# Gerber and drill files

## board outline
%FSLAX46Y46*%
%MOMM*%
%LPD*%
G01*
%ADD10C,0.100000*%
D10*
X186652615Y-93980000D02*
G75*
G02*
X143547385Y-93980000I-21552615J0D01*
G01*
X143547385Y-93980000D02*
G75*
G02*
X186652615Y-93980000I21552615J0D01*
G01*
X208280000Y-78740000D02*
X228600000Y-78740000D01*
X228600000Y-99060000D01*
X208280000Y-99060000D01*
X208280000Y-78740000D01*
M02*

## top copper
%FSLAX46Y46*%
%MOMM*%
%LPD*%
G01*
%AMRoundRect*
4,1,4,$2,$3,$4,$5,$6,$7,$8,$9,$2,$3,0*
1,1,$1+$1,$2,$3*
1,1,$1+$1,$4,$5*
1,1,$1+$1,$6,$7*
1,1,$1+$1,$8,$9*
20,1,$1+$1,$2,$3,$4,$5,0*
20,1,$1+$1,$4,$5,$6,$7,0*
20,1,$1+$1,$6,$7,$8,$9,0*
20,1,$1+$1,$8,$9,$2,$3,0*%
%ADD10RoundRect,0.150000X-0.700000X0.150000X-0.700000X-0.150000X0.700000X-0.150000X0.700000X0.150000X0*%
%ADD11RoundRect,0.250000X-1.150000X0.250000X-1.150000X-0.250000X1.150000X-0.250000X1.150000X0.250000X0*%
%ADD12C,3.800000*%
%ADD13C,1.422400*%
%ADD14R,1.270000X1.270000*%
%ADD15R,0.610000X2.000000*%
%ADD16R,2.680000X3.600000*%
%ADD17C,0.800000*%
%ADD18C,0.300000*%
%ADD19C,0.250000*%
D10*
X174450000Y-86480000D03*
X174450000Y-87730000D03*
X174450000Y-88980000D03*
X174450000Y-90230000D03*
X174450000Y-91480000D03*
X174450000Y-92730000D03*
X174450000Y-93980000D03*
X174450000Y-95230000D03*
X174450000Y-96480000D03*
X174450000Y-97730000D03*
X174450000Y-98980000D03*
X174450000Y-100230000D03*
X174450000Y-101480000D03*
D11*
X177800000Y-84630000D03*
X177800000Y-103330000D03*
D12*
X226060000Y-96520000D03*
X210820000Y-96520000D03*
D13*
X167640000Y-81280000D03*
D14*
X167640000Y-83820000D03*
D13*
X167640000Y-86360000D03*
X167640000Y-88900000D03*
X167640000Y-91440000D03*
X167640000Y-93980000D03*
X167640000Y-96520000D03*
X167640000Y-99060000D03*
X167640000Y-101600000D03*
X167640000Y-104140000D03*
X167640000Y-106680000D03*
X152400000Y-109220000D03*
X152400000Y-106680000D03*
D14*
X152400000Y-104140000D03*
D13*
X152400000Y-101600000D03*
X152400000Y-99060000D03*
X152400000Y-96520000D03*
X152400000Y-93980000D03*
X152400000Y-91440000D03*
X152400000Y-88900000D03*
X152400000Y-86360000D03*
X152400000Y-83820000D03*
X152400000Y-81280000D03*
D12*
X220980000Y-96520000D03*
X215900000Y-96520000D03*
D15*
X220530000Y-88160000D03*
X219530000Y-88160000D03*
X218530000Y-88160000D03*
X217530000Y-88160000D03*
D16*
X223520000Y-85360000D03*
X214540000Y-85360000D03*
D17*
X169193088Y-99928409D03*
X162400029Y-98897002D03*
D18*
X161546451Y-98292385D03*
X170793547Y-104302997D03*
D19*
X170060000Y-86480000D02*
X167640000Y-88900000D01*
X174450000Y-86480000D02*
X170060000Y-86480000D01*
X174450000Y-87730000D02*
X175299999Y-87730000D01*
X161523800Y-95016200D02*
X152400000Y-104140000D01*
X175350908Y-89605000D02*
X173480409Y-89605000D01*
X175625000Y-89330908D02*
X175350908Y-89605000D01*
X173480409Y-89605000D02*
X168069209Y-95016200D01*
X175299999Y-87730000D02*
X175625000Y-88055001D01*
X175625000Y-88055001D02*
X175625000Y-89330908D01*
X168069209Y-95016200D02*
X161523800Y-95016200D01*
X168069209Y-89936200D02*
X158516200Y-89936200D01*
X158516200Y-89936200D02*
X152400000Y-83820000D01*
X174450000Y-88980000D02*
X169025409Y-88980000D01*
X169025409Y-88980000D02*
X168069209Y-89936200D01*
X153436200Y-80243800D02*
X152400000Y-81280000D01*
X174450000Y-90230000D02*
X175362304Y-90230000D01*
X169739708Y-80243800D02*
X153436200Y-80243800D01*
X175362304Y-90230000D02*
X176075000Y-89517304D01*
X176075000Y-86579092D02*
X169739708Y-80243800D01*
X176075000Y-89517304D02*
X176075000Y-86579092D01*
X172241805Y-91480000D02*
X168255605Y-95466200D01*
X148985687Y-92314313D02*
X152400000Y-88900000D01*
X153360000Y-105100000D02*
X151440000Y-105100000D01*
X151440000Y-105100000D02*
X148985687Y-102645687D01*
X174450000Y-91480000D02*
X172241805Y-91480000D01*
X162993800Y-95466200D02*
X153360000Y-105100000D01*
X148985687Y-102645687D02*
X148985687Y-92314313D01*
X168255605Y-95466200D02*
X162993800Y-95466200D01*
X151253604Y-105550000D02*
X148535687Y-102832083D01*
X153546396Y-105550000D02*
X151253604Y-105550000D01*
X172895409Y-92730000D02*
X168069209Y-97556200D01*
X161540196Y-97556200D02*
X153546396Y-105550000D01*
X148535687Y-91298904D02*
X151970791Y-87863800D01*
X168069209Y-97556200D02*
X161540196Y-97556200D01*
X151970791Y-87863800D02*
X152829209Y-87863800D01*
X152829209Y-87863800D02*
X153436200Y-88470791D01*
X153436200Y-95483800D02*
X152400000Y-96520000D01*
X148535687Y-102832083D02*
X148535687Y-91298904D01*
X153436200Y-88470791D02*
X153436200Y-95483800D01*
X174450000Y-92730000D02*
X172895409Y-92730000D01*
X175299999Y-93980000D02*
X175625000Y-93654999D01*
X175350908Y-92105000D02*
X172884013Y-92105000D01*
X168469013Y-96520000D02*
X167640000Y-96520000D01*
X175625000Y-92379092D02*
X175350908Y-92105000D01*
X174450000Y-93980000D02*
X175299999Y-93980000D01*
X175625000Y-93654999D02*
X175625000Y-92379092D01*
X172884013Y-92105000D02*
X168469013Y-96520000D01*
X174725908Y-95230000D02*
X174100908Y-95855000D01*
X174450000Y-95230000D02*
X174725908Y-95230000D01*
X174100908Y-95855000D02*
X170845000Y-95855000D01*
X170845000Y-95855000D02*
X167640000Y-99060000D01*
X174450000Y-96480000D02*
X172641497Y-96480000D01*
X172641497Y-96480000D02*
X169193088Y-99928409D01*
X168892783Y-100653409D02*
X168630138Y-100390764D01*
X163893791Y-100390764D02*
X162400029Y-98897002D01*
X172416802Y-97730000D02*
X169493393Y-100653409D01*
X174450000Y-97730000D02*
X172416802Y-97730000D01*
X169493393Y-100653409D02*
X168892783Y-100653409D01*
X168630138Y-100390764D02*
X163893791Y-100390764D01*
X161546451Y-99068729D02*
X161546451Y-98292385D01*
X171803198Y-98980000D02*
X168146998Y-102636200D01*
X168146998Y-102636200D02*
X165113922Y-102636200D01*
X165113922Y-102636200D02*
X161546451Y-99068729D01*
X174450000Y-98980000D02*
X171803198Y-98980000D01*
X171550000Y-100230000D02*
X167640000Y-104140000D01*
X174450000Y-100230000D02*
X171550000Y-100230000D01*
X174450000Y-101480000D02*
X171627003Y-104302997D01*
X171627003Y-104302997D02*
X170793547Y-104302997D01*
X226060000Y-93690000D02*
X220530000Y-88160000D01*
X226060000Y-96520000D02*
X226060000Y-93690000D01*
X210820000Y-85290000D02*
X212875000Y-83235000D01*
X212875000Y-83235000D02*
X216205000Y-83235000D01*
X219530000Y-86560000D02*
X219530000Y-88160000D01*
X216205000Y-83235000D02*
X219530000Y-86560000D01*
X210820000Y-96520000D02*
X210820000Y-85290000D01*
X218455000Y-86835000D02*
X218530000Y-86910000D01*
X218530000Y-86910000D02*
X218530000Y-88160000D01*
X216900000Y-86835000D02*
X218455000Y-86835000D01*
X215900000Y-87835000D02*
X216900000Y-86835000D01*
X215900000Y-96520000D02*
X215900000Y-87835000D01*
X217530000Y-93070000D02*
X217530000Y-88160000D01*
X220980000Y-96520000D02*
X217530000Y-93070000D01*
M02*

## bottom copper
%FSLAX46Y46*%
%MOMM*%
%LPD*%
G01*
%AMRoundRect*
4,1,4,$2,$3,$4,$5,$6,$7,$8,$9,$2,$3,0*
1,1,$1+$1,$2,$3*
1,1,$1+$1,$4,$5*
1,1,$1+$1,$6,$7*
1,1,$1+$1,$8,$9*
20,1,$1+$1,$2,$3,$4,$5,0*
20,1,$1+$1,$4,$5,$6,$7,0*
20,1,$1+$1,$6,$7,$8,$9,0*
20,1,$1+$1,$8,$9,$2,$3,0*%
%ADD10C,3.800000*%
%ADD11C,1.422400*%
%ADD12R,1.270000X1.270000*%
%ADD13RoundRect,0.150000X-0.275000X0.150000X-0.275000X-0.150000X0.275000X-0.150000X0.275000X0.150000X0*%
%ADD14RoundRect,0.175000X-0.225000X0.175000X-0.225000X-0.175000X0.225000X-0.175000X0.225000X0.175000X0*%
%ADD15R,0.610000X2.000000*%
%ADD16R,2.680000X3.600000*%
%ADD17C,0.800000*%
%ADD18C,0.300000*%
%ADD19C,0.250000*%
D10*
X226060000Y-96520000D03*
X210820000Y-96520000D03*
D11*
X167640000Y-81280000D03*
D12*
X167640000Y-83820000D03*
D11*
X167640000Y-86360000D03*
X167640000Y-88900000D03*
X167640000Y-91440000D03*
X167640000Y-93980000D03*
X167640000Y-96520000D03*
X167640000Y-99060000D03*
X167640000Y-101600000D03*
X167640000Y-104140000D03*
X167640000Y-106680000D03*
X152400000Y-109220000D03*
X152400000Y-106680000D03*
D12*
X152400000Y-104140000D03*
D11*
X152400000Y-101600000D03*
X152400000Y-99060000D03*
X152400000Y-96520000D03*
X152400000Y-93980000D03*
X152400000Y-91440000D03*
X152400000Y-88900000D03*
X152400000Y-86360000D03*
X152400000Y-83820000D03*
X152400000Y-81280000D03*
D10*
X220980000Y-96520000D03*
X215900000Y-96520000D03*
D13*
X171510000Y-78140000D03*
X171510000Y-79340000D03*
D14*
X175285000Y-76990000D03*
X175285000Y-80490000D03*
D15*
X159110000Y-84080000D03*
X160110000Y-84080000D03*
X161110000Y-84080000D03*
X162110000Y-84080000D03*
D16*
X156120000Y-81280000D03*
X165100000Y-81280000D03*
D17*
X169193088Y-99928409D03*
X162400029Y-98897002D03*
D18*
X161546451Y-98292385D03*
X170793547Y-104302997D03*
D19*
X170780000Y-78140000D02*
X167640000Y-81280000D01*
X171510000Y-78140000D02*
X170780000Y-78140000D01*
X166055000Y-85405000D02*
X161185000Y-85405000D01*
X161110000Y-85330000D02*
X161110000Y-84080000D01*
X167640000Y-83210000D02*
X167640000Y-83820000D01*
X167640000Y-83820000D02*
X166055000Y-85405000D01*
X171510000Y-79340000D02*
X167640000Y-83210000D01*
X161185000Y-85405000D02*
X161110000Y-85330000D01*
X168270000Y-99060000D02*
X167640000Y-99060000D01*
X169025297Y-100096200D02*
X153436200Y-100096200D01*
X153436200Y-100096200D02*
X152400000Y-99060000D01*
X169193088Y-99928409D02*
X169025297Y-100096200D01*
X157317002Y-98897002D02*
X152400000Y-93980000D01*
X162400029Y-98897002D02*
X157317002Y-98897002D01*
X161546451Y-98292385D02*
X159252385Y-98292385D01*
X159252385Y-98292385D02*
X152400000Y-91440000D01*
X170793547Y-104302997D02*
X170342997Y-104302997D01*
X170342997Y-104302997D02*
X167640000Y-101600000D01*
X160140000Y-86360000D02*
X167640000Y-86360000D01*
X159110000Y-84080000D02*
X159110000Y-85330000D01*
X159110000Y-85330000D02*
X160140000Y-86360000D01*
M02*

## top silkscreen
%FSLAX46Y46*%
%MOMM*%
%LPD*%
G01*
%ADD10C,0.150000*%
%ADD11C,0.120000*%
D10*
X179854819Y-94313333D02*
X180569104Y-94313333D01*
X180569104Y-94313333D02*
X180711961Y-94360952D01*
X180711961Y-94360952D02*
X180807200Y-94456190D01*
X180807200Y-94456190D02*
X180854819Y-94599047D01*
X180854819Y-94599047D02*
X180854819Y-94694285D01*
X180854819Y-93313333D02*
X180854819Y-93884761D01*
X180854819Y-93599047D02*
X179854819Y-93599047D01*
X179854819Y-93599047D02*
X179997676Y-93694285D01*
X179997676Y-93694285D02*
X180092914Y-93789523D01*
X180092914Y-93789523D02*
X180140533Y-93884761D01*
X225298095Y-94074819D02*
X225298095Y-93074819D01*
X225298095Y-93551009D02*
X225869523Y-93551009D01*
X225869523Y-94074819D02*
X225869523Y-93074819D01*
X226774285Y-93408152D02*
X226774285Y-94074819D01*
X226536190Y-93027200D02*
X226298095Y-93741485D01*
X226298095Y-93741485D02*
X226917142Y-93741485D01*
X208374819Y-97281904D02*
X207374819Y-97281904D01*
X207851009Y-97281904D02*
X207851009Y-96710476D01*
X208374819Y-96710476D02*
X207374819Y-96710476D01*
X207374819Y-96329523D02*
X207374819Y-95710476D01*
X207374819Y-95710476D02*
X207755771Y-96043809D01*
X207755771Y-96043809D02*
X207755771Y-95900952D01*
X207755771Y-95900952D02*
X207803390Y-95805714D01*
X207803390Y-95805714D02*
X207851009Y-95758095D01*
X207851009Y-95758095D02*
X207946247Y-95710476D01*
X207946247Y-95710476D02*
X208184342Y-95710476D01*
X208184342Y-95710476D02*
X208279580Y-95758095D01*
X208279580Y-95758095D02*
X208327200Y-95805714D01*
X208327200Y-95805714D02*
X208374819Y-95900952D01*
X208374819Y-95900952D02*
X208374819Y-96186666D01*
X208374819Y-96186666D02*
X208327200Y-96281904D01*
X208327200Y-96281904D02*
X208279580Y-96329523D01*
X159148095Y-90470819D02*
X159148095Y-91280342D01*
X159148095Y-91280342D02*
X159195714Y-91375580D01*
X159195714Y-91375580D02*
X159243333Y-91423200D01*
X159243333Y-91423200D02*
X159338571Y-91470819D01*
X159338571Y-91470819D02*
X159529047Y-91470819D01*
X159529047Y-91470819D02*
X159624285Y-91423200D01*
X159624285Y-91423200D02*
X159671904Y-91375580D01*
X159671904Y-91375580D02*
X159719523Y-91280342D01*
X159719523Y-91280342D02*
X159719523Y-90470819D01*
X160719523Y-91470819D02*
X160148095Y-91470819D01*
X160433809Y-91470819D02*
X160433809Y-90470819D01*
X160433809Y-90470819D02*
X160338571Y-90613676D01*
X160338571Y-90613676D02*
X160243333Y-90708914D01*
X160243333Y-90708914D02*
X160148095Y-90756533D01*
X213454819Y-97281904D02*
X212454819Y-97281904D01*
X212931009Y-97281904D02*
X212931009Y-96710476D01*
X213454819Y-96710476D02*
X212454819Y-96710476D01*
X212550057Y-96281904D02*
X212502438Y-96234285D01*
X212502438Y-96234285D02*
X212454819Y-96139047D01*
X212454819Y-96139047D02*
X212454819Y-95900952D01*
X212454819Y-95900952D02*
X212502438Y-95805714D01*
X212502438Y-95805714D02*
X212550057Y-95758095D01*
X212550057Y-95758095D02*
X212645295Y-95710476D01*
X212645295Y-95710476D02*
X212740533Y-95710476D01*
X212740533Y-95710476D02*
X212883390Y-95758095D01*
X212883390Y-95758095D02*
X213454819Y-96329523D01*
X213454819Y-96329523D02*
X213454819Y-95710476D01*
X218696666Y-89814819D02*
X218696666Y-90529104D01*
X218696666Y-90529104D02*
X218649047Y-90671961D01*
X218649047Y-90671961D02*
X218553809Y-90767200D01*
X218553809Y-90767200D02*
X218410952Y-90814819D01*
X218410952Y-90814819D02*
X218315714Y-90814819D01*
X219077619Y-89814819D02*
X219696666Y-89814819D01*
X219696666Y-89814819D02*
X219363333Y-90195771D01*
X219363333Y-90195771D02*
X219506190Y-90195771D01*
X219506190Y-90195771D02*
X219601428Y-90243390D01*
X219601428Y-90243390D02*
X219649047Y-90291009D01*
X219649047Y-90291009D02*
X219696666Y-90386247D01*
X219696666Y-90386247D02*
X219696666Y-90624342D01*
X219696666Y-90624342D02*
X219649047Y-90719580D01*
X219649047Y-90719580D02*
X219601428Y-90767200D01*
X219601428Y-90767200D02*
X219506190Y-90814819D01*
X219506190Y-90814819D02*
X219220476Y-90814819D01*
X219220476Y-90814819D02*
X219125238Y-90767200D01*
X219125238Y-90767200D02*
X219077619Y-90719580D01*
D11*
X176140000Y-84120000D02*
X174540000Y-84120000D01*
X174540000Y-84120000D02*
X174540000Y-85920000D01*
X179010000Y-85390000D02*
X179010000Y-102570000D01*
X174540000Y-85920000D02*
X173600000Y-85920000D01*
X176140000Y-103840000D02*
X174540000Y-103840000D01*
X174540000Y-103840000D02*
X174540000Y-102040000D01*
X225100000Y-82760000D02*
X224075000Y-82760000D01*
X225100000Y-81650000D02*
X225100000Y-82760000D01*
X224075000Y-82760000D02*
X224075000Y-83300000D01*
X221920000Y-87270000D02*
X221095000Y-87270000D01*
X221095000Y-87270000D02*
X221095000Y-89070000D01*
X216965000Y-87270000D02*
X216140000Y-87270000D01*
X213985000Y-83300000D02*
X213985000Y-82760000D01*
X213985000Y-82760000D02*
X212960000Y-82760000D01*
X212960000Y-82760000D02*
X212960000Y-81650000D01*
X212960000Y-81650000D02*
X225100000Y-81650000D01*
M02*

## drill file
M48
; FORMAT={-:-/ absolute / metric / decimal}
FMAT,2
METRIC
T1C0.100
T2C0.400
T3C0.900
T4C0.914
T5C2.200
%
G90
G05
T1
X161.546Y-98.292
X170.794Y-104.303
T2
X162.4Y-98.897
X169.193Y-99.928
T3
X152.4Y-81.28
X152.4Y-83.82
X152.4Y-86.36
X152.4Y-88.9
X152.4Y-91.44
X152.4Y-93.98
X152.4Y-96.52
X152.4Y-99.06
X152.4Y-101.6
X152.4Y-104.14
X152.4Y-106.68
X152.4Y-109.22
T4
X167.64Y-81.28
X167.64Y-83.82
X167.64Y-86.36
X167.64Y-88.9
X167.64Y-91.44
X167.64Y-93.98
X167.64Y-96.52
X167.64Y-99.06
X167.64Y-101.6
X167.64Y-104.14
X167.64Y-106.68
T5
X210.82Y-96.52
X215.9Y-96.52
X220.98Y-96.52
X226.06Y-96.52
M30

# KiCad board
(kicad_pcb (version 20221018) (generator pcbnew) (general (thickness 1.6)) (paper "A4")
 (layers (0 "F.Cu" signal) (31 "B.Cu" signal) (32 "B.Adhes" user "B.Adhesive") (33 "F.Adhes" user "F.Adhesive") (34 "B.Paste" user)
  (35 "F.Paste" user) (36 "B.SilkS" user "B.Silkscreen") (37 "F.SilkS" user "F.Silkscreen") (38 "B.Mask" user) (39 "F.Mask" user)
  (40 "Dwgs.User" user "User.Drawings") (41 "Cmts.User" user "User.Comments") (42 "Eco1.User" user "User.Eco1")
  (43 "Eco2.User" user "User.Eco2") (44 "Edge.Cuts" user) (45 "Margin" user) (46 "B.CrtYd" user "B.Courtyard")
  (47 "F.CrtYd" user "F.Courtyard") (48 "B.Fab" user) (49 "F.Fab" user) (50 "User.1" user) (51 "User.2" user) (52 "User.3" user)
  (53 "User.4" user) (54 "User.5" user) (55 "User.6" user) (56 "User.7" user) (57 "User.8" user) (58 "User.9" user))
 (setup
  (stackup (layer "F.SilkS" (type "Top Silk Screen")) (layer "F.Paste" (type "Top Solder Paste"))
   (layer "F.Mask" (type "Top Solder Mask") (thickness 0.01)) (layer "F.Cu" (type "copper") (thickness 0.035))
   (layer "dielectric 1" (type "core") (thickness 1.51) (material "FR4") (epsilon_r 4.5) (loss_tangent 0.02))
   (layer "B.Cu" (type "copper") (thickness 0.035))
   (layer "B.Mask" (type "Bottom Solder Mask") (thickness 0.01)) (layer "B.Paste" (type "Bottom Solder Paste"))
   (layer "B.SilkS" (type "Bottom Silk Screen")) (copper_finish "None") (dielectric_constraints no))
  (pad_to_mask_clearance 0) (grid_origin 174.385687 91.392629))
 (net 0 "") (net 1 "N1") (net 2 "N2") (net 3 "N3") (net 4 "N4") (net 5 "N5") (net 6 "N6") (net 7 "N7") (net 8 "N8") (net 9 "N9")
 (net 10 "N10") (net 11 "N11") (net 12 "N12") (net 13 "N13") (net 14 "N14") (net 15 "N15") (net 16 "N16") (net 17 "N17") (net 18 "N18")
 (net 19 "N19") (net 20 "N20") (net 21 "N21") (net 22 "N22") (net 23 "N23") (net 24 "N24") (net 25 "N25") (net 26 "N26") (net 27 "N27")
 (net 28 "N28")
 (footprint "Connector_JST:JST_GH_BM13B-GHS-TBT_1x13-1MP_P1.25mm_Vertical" (layer "F.Cu") (at 176.4 93.98 -90)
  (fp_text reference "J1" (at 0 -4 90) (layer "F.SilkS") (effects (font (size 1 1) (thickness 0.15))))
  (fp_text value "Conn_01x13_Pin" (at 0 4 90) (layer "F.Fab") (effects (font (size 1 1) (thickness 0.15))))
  (fp_line (start -9.86 0.26) (end -9.86 1.86) (stroke (width 0.12) (type solid)) (layer "F.SilkS"))
  (fp_line (start -9.86 1.86) (end -8.06 1.86) (stroke (width 0.12) (type solid)) (layer "F.SilkS"))
  (fp_line (start -8.59 -2.61) (end 8.59 -2.61) (stroke (width 0.12) (type solid)) (layer "F.SilkS"))
  (fp_line (start -8.06 1.86) (end -8.06 2.8) (stroke (width 0.12) (type solid)) (layer "F.SilkS"))
  (fp_line (start 9.86 0.26) (end 9.86 1.86) (stroke (width 0.12) (type solid)) (layer "F.SilkS"))
  (fp_line (start 9.86 1.86) (end 8.06 1.86) (stroke (width 0.12) (type solid)) (layer "F.SilkS"))
  (pad "1" smd roundrect (at -7.5 1.95 270) (size 0.6 1.7) (layers "F.Cu" "F.Paste" "F.Mask") (roundrect_rratio 0.25) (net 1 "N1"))
  (pad "2" smd roundrect (at -6.25 1.95 270) (size 0.6 1.7) (layers "F.Cu" "F.Paste" "F.Mask") (roundrect_rratio 0.25) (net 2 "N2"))
  (pad "3" smd roundrect (at -5 1.95 270) (size 0.6 1.7) (layers "F.Cu" "F.Paste" "F.Mask") (roundrect_rratio 0.25) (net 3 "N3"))
  (pad "4" smd roundrect (at -3.75 1.95 270) (size 0.6 1.7) (layers "F.Cu" "F.Paste" "F.Mask") (roundrect_rratio 0.25) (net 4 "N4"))
  (pad "5" smd roundrect (at -2.5 1.95 270) (size 0.6 1.7) (layers "F.Cu" "F.Paste" "F.Mask") (roundrect_rratio 0.25) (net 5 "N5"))
  (pad "6" smd roundrect (at -1.25 1.95 270) (size 0.6 1.7) (layers "F.Cu" "F.Paste" "F.Mask") (roundrect_rratio 0.25) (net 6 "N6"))
  (pad "7" smd roundrect (at 0 1.95 270) (size 0.6 1.7) (layers "F.Cu" "F.Paste" "F.Mask") (roundrect_rratio 0.25) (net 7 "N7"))
  (pad "8" smd roundrect (at 1.25 1.95 270) (size 0.6 1.7) (layers "F.Cu" "F.Paste" "F.Mask") (roundrect_rratio 0.25) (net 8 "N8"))
  (pad "9" smd roundrect (at 2.5 1.95 270) (size 0.6 1.7) (layers "F.Cu" "F.Paste" "F.Mask") (roundrect_rratio 0.25) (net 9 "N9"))
  (pad "10" smd roundrect (at 3.75 1.95 270) (size 0.6 1.7) (layers "F.Cu" "F.Paste" "F.Mask") (roundrect_rratio 0.25) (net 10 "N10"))
  (pad "11" smd roundrect (at 5 1.95 270) (size 0.6 1.7) (layers "F.Cu" "F.Paste" "F.Mask") (roundrect_rratio 0.25) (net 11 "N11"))
  (pad "12" smd roundrect (at 6.25 1.95 270) (size 0.6 1.7) (layers "F.Cu" "F.Paste" "F.Mask") (roundrect_rratio 0.25) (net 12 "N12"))
  (pad "13" smd roundrect (at 7.5 1.95 270) (size 0.6 1.7) (layers "F.Cu" "F.Paste" "F.Mask") (roundrect_rratio 0.25) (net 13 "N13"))
  (pad "MP" smd roundrect (at -9.35 -1.4 270) (size 1 2.8) (layers "F.Cu" "F.Paste" "F.Mask") (roundrect_rratio 0.25))
  (pad "MP" smd roundrect (at 9.35 -1.4 270) (size 1 2.8) (layers "F.Cu" "F.Paste" "F.Mask") (roundrect_rratio 0.25)))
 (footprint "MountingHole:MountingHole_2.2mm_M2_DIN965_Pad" (layer "F.Cu") (at 226.06 96.52)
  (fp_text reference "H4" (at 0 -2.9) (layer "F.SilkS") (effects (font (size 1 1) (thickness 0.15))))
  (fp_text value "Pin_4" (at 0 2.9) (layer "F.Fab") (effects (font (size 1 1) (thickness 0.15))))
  (pad "1" thru_hole circle (at 0 0) (size 3.8 3.8) (drill 2.2) (layers "*.Cu" "*.Mask") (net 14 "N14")))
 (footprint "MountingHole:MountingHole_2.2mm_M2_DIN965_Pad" (layer "F.Cu") (at 210.82 96.52 90)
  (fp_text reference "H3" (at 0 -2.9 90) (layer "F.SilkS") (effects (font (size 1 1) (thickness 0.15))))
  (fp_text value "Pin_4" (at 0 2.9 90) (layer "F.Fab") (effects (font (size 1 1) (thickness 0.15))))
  (pad "1" thru_hole circle (at 0 0 90) (size 3.8 3.8) (drill 2.2) (layers "*.Cu" "*.Mask") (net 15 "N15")))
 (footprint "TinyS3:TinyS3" (layer "F.Cu") (at 159.91 95.216)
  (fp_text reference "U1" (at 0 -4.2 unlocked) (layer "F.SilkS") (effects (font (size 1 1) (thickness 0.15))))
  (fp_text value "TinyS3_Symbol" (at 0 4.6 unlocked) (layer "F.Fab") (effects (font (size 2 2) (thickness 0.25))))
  (pad "1" thru_hole circle (at 7.73 -13.936) (size 1.4224 1.4224) (drill 0.9144) (layers "*.Cu" "*.Mask") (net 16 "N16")
   (solder_mask_margin 0.0254))
  (pad "2" thru_hole rect (at 7.73 -11.396) (size 1.27 1.27) (drill 0.9144) (layers "*.Cu" "*.Mask") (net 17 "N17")
   (solder_mask_margin 0.0254))
  (pad "3" thru_hole circle (at 7.73 -8.856) (size 1.4224 1.4224) (drill 0.9144) (layers "*.Cu" "*.Mask") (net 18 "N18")
   (solder_mask_margin 0.0254))
  (pad "4" thru_hole circle (at 7.73 -6.316) (size 1.4224 1.4224) (drill 0.9144) (layers "*.Cu" "*.Mask") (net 1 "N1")
   (solder_mask_margin 0.0254))
  (pad "5" thru_hole circle (at 7.73 -3.776) (size 1.4224 1.4224) (drill 0.9144) (layers "*.Cu" "*.Mask") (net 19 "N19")
   (solder_mask_margin 0.0254))
  (pad "6" thru_hole circle (at 7.73 -1.236) (size 1.4224 1.4224) (drill 0.9144) (layers "*.Cu" "*.Mask") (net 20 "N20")
   (solder_mask_margin 0.0254))
  (pad "7" thru_hole circle (at 7.73 1.304) (size 1.4224 1.4224) (drill 0.9144) (layers "*.Cu" "*.Mask") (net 7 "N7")
   (solder_mask_margin 0.0254))
  (pad "8" thru_hole circle (at 7.73 3.844) (size 1.4224 1.4224) (drill 0.9144) (layers "*.Cu" "*.Mask") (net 8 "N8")
   (solder_mask_margin 0.0254))
  (pad "9" thru_hole circle (at 7.73 6.384) (size 1.4224 1.4224) (drill 0.9144) (layers "*.Cu" "*.Mask") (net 13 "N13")
   (solder_mask_margin 0.0254))
  (pad "10" thru_hole circle (at 7.73 8.924) (size 1.4224 1.4224) (drill 0.9144) (layers "*.Cu" "*.Mask") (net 12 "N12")
   (solder_mask_margin 0.0254))
  (pad "11" thru_hole circle (at 7.73 11.464) (size 1.4224 1.4224) (drill 0.9144) (layers "*.Cu" "*.Mask") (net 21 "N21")
   (solder_mask_margin 0.0254))
  (pad "12" thru_hole circle (at -7.51 14.004) (size 1.4224 1.4224) (drill 0.9) (layers "*.Cu" "*.Mask") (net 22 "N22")
   (solder_mask_margin 0.0254))
  (pad "13" thru_hole circle (at -7.51 11.464) (size 1.4224 1.4224) (drill 0.9) (layers "*.Cu" "*.Mask") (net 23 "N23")
   (solder_mask_margin 0.0254))
  (pad "14" thru_hole rect (at -7.51 8.924) (size 1.27 1.27) (drill 0.9) (layers "*.Cu" "*.Mask") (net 2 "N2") (solder_mask_margin 0.0254))
  (pad "15" thru_hole circle (at -7.51 6.384) (size 1.4224 1.4224) (drill 0.9) (layers "*.Cu" "*.Mask") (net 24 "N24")
   (solder_mask_margin 0.0254))
  (pad "16" thru_hole circle (at -7.51 3.844) (size 1.4224 1.4224) (drill 0.9) (layers "*.Cu" "*.Mask") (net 9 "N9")
   (solder_mask_margin 0.0254))
  (pad "17" thru_hole circle (at -7.51 1.304) (size 1.4224 1.4224) (drill 0.9) (layers "*.Cu" "*.Mask") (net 6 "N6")
   (solder_mask_margin 0.0254))
  (pad "18" thru_hole circle (at -7.51 -1.236) (size 1.4224 1.4224) (drill 0.9) (layers "*.Cu" "*.Mask") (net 10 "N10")
   (solder_mask_margin 0.0254))
  (pad "19" thru_hole circle (at -7.51 -3.776) (size 1.4224 1.4224) (drill 0.9) (layers "*.Cu" "*.Mask") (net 11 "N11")
   (solder_mask_margin 0.0254))
  (pad "20" thru_hole circle (at -7.51 -6.316) (size 1.4224 1.4224) (drill 0.9) (layers "*.Cu" "*.Mask") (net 5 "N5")
   (solder_mask_margin 0.0254))
  (pad "21" thru_hole circle (at -7.51 -8.856) (size 1.4224 1.4224) (drill 0.9) (layers "*.Cu" "*.Mask") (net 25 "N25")
   (solder_mask_margin 0.0254))
  (pad "22" thru_hole circle (at -7.51 -11.396) (size 1.4224 1.4224) (drill 0.9) (layers "*.Cu" "*.Mask") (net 3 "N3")
   (solder_mask_margin 0.0254))
  (pad "23" thru_hole circle (at -7.51 -13.936) (size 1.4224 1.4224) (drill 0.9) (layers "*.Cu" "*.Mask") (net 4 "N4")
   (solder_mask_margin 0.0254)))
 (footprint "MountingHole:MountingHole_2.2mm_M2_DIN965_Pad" (layer "F.Cu") (at 220.98 96.52 90)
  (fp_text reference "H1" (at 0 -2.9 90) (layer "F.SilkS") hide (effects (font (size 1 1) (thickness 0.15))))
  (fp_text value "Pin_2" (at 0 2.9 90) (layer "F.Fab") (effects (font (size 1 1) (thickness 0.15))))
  (pad "1" thru_hole circle (at 0 0 90) (size 3.8 3.8) (drill 2.2) (layers "*.Cu" "*.Mask") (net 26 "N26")))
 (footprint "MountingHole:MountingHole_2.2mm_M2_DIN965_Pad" (layer "F.Cu") (at 215.9 96.52 90)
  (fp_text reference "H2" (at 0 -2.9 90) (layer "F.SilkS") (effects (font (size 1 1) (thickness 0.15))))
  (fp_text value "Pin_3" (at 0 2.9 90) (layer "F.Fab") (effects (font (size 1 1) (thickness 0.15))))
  (pad "1" thru_hole circle (at 0 0 90) (size 3.8 3.8) (drill 2.2) (layers "*.Cu" "*.Mask") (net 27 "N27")))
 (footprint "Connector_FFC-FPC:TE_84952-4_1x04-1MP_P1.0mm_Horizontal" (layer "F.Cu") (at 219.03 86.36 180)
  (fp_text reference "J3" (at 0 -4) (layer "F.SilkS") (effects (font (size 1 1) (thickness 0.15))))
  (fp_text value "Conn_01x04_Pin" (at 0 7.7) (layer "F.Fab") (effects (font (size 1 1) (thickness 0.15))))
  (fp_line (start -6.07 3.6) (end -5.045 3.6) (stroke (width 0.12) (type solid)) (layer "F.SilkS"))
  (fp_line (start -6.07 4.71) (end -6.07 3.6) (stroke (width 0.12) (type solid)) (layer "F.SilkS"))
  (fp_line (start -5.045 3.6) (end -5.045 3.06) (stroke (width 0.12) (type solid)) (layer "F.SilkS"))
  (fp_line (start -2.89 -0.91) (end -2.065 -0.91) (stroke (width 0.12) (type solid)) (layer "F.SilkS"))
  (fp_line (start -2.065 -0.91) (end -2.065 -2.71) (stroke (width 0.12) (type solid)) (layer "F.SilkS"))
  (fp_line (start 2.065 -0.91) (end 2.89 -0.91) (stroke (width 0.12) (type solid)) (layer "F.SilkS"))
  (fp_line (start 5.045 3.06) (end 5.045 3.6) (stroke (width 0.12) (type solid)) (layer "F.SilkS"))
  (fp_line (start 5.045 3.6) (end 6.07 3.6) (stroke (width 0.12) (type solid)) (layer "F.SilkS"))
  (fp_line (start 6.07 3.6) (end 6.07 4.71) (stroke (width 0.12) (type solid)) (layer "F.SilkS"))
  (fp_line (start 6.07 4.71) (end -6.07 4.71) (stroke (width 0.12) (type solid)) (layer "F.SilkS"))
  (pad "1" smd rect (at -1.5 -1.8 180) (size 0.61 2) (layers "F.Cu" "F.Paste" "F.Mask") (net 14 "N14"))
  (pad "2" smd rect (at -0.5 -1.8 180) (size 0.61 2) (layers "F.Cu" "F.Paste" "F.Mask") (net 15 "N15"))
  (pad "3" smd rect (at 0.5 -1.8 180) (size 0.61 2) (layers "F.Cu" "F.Paste" "F.Mask") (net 27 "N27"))
  (pad "4" smd rect (at 1.5 -1.8 180) (size 0.61 2) (layers "F.Cu" "F.Paste" "F.Mask") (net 26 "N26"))
  (pad "MP" smd rect (at -4.49 1 180) (size 2.68 3.6) (layers "F.Cu" "F.Paste" "F.Mask"))
  (pad "MP" smd rect (at 4.49 1 180) (size 2.68 3.6) (layers "F.Cu" "F.Paste" "F.Mask")))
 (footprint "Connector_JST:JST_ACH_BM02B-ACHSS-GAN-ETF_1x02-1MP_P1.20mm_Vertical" (layer "B.Cu") (at 173.385 78.74 -90)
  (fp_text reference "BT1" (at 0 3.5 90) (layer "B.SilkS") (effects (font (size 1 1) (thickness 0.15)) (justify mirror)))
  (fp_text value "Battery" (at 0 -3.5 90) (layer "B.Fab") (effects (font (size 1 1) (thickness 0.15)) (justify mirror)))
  (pad "1" smd roundrect (at -0.6 1.875 270) (size 0.6 0.85) (layers "B.Cu" "B.Paste" "B.Mask") (roundrect_rratio 0.25) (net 16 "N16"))
  (pad "2" smd roundrect (at 0.6 1.875 270) (size 0.6 0.85) (layers "B.Cu" "B.Paste" "B.Mask") (roundrect_rratio 0.25) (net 17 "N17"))
  (pad "MP" smd roundrect (at -1.75 -1.9 270) (size 0.7 0.8) (layers "B.Cu" "B.Paste" "B.Mask") (roundrect_rratio 0.25))
  (pad "MP" smd roundrect (at 1.75 -1.9 270) (size 0.7 0.8) (layers "B.Cu" "B.Paste" "B.Mask") (roundrect_rratio 0.25)))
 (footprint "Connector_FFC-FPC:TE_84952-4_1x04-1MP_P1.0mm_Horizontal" (layer "B.Cu") (at 160.61 82.28)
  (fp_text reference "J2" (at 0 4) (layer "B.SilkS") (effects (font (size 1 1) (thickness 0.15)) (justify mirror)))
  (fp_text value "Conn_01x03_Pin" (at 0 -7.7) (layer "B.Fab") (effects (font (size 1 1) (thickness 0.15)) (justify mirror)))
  (pad "1" smd rect (at -1.5 1.8) (size 0.61 2) (layers "B.Cu" "B.Paste" "B.Mask") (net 18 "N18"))
  (pad "2" smd rect (at -0.5 1.8) (size 0.61 2) (layers "B.Cu" "B.Paste" "B.Mask") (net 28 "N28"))
  (pad "3" smd rect (at 0.5 1.8) (size 0.61 2) (layers "B.Cu" "B.Paste" "B.Mask") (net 17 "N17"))
  (pad "4" smd rect (at 1.5 1.8) (size 0.61 2) (layers "B.Cu" "B.Paste" "B.Mask"))
  (pad "MP" smd rect (at -4.49 -1) (size 2.68 3.6) (layers "B.Cu" "B.Paste" "B.Mask"))
  (pad "MP" smd rect (at 4.49 -1) (size 2.68 3.6) (layers "B.Cu" "B.Paste" "B.Mask")))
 (gr_circle (center 165.1 93.98) (end 180.34 78.74) (stroke (width 0.1) (type default)) (fill none) (layer "Edge.Cuts"))
 (gr_rect (start 208.28 78.74) (end 228.6 99.06) (stroke (width 0.1) (type default)) (fill none) (layer "Edge.Cuts"))
 (segment (start 170.78 78.14) (end 167.64 81.28) (width 0.25) (layer "B.Cu") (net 16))
 (segment (start 171.51 78.14) (end 170.78 78.14) (width 0.25) (layer "B.Cu") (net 16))
 (segment (start 166.055 85.405) (end 161.185 85.405) (width 0.25) (layer "B.Cu") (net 17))
 (segment (start 161.11 85.33) (end 161.11 84.08) (width 0.25) (layer "B.Cu") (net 17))
 (segment (start 167.64 83.21) (end 167.64 83.82) (width 0.25) (layer "B.Cu") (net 17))
 (segment (start 167.64 83.82) (end 166.055 85.405) (width 0.25) (layer "B.Cu") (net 17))
 (segment (start 171.51 79.34) (end 167.64 83.21) (width 0.25) (layer "B.Cu") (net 17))
 (segment (start 161.185 85.405) (end 161.11 85.33) (width 0.25) (layer "B.Cu") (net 17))
 (segment (start 170.06 86.48) (end 167.64 88.9) (width 0.25) (layer "F.Cu") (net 1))
 (segment (start 174.45 86.48) (end 170.06 86.48) (width 0.25) (layer "F.Cu") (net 1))
 (segment (start 174.45 87.73) (end 175.299999 87.73) (width 0.25) (layer "F.Cu") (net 2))
 (segment (start 161.5238 95.0162) (end 152.4 104.14) (width 0.25) (layer "F.Cu") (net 2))
 (segment (start 175.350908 89.605) (end 173.480409 89.605) (width 0.25) (layer "F.Cu") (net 2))
 (segment (start 175.625 89.330908) (end 175.350908 89.605) (width 0.25) (layer "F.Cu") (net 2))
 (segment (start 173.480409 89.605) (end 168.069209 95.0162) (width 0.25) (layer "F.Cu") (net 2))
 (segment (start 175.299999 87.73) (end 175.625 88.055001) (width 0.25) (layer "F.Cu") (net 2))
 (segment (start 175.625 88.055001) (end 175.625 89.330908) (width 0.25) (layer "F.Cu") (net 2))
 (segment (start 168.069209 95.0162) (end 161.5238 95.0162) (width 0.25) (layer "F.Cu") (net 2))
 (segment (start 168.069209 89.9362) (end 158.5162 89.9362) (width 0.25) (layer "F.Cu") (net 3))
 (segment (start 158.5162 89.9362) (end 152.4 83.82) (width 0.25) (layer "F.Cu") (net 3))
 (segment (start 174.45 88.98) (end 169.025409 88.98) (width 0.25) (layer "F.Cu") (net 3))
 (segment (start 169.025409 88.98) (end 168.069209 89.9362) (width 0.25) (layer "F.Cu") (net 3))
 (segment (start 153.4362 80.2438) (end 152.4 81.28) (width 0.25) (layer "F.Cu") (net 4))
 (segment (start 174.45 90.23) (end 175.362304 90.23) (width 0.25) (layer "F.Cu") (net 4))
 (segment (start 169.739708 80.2438) (end 153.4362 80.2438) (width 0.25) (layer "F.Cu") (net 4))
 (segment (start 175.362304 90.23) (end 176.075 89.517304) (width 0.25) (layer "F.Cu") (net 4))
 (segment (start 176.075 86.579092) (end 169.739708 80.2438) (width 0.25) (layer "F.Cu") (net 4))
 (segment (start 176.075 89.517304) (end 176.075 86.579092) (width 0.25) (layer "F.Cu") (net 4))
 (segment (start 172.241805 91.48) (end 168.255605 95.4662) (width 0.25) (layer "F.Cu") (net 5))
 (segment (start 148.985687 92.314313) (end 152.4 88.9) (width 0.25) (layer "F.Cu") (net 5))
 (segment (start 153.36 105.1) (end 151.44 105.1) (width 0.25) (layer "F.Cu") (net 5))
 (segment (start 151.44 105.1) (end 148.985687 102.645687) (width 0.25) (layer "F.Cu") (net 5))
 (segment (start 174.45 91.48) (end 172.241805 91.48) (width 0.25) (layer "F.Cu") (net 5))
 (segment (start 162.9938 95.4662) (end 153.36 105.1) (width 0.25) (layer "F.Cu") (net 5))
 (segment (start 148.985687 102.645687) (end 148.985687 92.314313) (width 0.25) (layer "F.Cu") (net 5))
 (segment (start 168.255605 95.4662) (end 162.9938 95.4662) (width 0.25) (layer "F.Cu") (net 5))
 (segment (start 151.253604 105.55) (end 148.535687 102.832083) (width 0.25) (layer "F.Cu") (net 6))
 (segment (start 153.546396 105.55) (end 151.253604 105.55) (width 0.25) (layer "F.Cu") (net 6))
 (segment (start 172.895409 92.73) (end 168.069209 97.5562) (width 0.25) (layer "F.Cu") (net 6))
 (segment (start 161.540196 97.5562) (end 153.546396 105.55) (width 0.25) (layer "F.Cu") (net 6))
 (segment (start 148.535687 91.298904) (end 151.970791 87.8638) (width 0.25) (layer "F.Cu") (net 6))
 (segment (start 168.069209 97.5562) (end 161.540196 97.5562) (width 0.25) (layer "F.Cu") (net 6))
 (segment (start 151.970791 87.8638) (end 152.829209 87.8638) (width 0.25) (layer "F.Cu") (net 6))
 (segment (start 152.829209 87.8638) (end 153.4362 88.470791) (width 0.25) (layer "F.Cu") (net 6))
 (segment (start 153.4362 95.4838) (end 152.4 96.52) (width 0.25) (layer "F.Cu") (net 6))
 (segment (start 148.535687 102.832083) (end 148.535687 91.298904) (width 0.25) (layer "F.Cu") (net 6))
 (segment (start 153.4362 88.470791) (end 153.4362 95.4838) (width 0.25) (layer "F.Cu") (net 6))
 (segment (start 174.45 92.73) (end 172.895409 92.73) (width 0.25) (layer "F.Cu") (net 6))
 (segment (start 175.299999 93.98) (end 175.625 93.654999) (width 0.25) (layer "F.Cu") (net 7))
 (segment (start 175.350908 92.105) (end 172.884013 92.105) (width 0.25) (layer "F.Cu") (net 7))
 (segment (start 168.469013 96.52) (end 167.64 96.52) (width 0.25) (layer "F.Cu") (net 7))
 (segment (start 175.625 92.379092) (end 175.350908 92.105) (width 0.25) (layer "F.Cu") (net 7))
 (segment (start 174.45 93.98) (end 175.299999 93.98) (width 0.25) (layer "F.Cu") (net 7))
 (segment (start 175.625 93.654999) (end 175.625 92.379092) (width 0.25) (layer "F.Cu") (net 7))
 (segment (start 172.884013 92.105) (end 168.469013 96.52) (width 0.25) (layer "F.Cu") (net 7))
 (segment (start 174.725908 95.23) (end 174.100908 95.855) (width 0.25) (layer "F.Cu") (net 8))
 (segment (start 174.45 95.23) (end 174.725908 95.23) (width 0.25) (layer "F.Cu") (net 8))
 (segment (start 174.100908 95.855) (end 170.845 95.855) (width 0.25) (layer "F.Cu") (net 8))
 (segment (start 170.845 95.855) (end 167.64 99.06) (width 0.25) (layer "F.Cu") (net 8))
 (segment (start 168.27 99.06) (end 167.64 99.06) (width 0.25) (layer "B.Cu") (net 8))
 (segment (start 174.45 96.48) (end 172.641497 96.48) (width 0.25) (layer "F.Cu") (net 9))
 (segment (start 172.641497 96.48) (end 169.193088 99.928409) (width 0.25) (layer "F.Cu") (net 9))
 (via (at 169.193088 99.928409) (size 0.8) (drill 0.4) (layers "F.Cu" "B.Cu") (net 9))
 (segment (start 169.025297 100.0962) (end 153.4362 100.0962) (width 0.25) (layer "B.Cu") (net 9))
 (segment (start 153.4362 100.0962) (end 152.4 99.06) (width 0.25) (layer "B.Cu") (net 9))
 (segment (start 169.193088 99.928409) (end 169.025297 100.0962) (width 0.25) (layer "B.Cu") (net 9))
 (segment (start 168.892783 100.653409) (end 168.630138 100.390764) (width 0.25) (layer "F.Cu") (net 10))
 (segment (start 163.893791 100.390764) (end 162.400029 98.897002) (width 0.25) (layer "F.Cu") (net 10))
 (segment (start 172.416802 97.73) (end 169.493393 100.653409) (width 0.25) (layer "F.Cu") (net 10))
 (segment (start 174.45 97.73) (end 172.416802 97.73) (width 0.25) (layer "F.Cu") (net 10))
 (segment (start 169.493393 100.653409) (end 168.892783 100.653409) (width 0.25) (layer "F.Cu") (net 10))
 (segment (start 168.630138 100.390764) (end 163.893791 100.390764) (width 0.25) (layer "F.Cu") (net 10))
 (via (at 162.400029 98.897002) (size 0.8) (drill 0.4) (layers "F.Cu" "B.Cu") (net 10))
 (segment (start 157.317002 98.897002) (end 152.4 93.98) (width 0.25) (layer "B.Cu") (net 10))
 (segment (start 162.400029 98.897002) (end 157.317002 98.897002) (width 0.25) (layer "B.Cu") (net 10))
 (segment (start 161.546451 99.068729) (end 161.546451 98.292385) (width 0.25) (layer "F.Cu") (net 11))
 (segment (start 171.803198 98.98) (end 168.146998 102.6362) (width 0.25) (layer "F.Cu") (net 11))
 (segment (start 168.146998 102.6362) (end 165.113922 102.6362) (width 0.25) (layer "F.Cu") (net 11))
 (segment (start 165.113922 102.6362) (end 161.546451 99.068729) (width 0.25) (layer "F.Cu") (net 11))
 (segment (start 174.45 98.98) (end 171.803198 98.98) (width 0.25) (layer "F.Cu") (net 11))
 (via micro (at 161.546451 98.292385) (size 0.3) (drill 0.1) (layers "F.Cu" "B.Cu") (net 11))
 (segment (start 161.546451 98.292385) (end 159.252385 98.292385) (width 0.25) (layer "B.Cu") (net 11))
 (segment (start 159.252385 98.292385) (end 152.4 91.44) (width 0.25) (layer "B.Cu") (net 11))
 (segment (start 171.55 100.23) (end 167.64 104.14) (width 0.25) (layer "F.Cu") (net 12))
 (segment (start 174.45 100.23) (end 171.55 100.23) (width 0.25) (layer "F.Cu") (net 12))
 (segment (start 174.45 101.48) (end 171.627003 104.302997) (width 0.25) (layer "F.Cu") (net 13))
 (segment (start 171.627003 104.302997) (end 170.793547 104.302997) (width 0.25) (layer "F.Cu") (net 13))
 (via micro (at 170.793547 104.302997) (size 0.3) (drill 0.1) (layers "F.Cu" "B.Cu") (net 13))
 (segment (start 170.793547 104.302997) (end 170.342997 104.302997) (width 0.25) (layer "B.Cu") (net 13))
 (segment (start 170.342997 104.302997) (end 167.64 101.6) (width 0.25) (layer "B.Cu") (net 13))
 (segment (start 160.14 86.36) (end 167.64 86.36) (width 0.25) (layer "B.Cu") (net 18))
 (segment (start 159.11 84.08) (end 159.11 85.33) (width 0.25) (layer "B.Cu") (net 18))
 (segment (start 159.11 85.33) (end 160.14 86.36) (width 0.25) (layer "B.Cu") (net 18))
 (segment (start 226.06 93.69) (end 220.53 88.16) (width 0.25) (layer "F.Cu") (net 14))
 (segment (start 226.06 96.52) (end 226.06 93.69) (width 0.25) (layer "F.Cu") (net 14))
 (segment (start 210.82 85.29) (end 212.875 83.235) (width 0.25) (layer "F.Cu") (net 15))
 (segment (start 212.875 83.235) (end 216.205 83.235) (width 0.25) (layer "F.Cu") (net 15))
 (segment (start 219.53 86.56) (end 219.53 88.16) (width 0.25) (layer "F.Cu") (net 15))
 (segment (start 216.205 83.235) (end 219.53 86.56) (width 0.25) (layer "F.Cu") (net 15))
 (segment (start 210.82 96.52) (end 210.82 85.29) (width 0.25) (layer "F.Cu") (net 15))
 (segment (start 218.455 86.835) (end 218.53 86.91) (width 0.25) (layer "F.Cu") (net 27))
 (segment (start 218.53 86.91) (end 218.53 88.16) (width 0.25) (layer "F.Cu") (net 27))
 (segment (start 216.9 86.835) (end 218.455 86.835) (width 0.25) (layer "F.Cu") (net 27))
 (segment (start 215.9 87.835) (end 216.9 86.835) (width 0.25) (layer "F.Cu") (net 27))
 (segment (start 215.9 96.52) (end 215.9 87.835) (width 0.25) (layer "F.Cu") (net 27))
 (segment (start 217.53 93.07) (end 217.53 88.16) (width 0.25) (layer "F.Cu") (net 26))
 (segment (start 220.98 96.52) (end 217.53 93.07) (width 0.25) (layer "F.Cu") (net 26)))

